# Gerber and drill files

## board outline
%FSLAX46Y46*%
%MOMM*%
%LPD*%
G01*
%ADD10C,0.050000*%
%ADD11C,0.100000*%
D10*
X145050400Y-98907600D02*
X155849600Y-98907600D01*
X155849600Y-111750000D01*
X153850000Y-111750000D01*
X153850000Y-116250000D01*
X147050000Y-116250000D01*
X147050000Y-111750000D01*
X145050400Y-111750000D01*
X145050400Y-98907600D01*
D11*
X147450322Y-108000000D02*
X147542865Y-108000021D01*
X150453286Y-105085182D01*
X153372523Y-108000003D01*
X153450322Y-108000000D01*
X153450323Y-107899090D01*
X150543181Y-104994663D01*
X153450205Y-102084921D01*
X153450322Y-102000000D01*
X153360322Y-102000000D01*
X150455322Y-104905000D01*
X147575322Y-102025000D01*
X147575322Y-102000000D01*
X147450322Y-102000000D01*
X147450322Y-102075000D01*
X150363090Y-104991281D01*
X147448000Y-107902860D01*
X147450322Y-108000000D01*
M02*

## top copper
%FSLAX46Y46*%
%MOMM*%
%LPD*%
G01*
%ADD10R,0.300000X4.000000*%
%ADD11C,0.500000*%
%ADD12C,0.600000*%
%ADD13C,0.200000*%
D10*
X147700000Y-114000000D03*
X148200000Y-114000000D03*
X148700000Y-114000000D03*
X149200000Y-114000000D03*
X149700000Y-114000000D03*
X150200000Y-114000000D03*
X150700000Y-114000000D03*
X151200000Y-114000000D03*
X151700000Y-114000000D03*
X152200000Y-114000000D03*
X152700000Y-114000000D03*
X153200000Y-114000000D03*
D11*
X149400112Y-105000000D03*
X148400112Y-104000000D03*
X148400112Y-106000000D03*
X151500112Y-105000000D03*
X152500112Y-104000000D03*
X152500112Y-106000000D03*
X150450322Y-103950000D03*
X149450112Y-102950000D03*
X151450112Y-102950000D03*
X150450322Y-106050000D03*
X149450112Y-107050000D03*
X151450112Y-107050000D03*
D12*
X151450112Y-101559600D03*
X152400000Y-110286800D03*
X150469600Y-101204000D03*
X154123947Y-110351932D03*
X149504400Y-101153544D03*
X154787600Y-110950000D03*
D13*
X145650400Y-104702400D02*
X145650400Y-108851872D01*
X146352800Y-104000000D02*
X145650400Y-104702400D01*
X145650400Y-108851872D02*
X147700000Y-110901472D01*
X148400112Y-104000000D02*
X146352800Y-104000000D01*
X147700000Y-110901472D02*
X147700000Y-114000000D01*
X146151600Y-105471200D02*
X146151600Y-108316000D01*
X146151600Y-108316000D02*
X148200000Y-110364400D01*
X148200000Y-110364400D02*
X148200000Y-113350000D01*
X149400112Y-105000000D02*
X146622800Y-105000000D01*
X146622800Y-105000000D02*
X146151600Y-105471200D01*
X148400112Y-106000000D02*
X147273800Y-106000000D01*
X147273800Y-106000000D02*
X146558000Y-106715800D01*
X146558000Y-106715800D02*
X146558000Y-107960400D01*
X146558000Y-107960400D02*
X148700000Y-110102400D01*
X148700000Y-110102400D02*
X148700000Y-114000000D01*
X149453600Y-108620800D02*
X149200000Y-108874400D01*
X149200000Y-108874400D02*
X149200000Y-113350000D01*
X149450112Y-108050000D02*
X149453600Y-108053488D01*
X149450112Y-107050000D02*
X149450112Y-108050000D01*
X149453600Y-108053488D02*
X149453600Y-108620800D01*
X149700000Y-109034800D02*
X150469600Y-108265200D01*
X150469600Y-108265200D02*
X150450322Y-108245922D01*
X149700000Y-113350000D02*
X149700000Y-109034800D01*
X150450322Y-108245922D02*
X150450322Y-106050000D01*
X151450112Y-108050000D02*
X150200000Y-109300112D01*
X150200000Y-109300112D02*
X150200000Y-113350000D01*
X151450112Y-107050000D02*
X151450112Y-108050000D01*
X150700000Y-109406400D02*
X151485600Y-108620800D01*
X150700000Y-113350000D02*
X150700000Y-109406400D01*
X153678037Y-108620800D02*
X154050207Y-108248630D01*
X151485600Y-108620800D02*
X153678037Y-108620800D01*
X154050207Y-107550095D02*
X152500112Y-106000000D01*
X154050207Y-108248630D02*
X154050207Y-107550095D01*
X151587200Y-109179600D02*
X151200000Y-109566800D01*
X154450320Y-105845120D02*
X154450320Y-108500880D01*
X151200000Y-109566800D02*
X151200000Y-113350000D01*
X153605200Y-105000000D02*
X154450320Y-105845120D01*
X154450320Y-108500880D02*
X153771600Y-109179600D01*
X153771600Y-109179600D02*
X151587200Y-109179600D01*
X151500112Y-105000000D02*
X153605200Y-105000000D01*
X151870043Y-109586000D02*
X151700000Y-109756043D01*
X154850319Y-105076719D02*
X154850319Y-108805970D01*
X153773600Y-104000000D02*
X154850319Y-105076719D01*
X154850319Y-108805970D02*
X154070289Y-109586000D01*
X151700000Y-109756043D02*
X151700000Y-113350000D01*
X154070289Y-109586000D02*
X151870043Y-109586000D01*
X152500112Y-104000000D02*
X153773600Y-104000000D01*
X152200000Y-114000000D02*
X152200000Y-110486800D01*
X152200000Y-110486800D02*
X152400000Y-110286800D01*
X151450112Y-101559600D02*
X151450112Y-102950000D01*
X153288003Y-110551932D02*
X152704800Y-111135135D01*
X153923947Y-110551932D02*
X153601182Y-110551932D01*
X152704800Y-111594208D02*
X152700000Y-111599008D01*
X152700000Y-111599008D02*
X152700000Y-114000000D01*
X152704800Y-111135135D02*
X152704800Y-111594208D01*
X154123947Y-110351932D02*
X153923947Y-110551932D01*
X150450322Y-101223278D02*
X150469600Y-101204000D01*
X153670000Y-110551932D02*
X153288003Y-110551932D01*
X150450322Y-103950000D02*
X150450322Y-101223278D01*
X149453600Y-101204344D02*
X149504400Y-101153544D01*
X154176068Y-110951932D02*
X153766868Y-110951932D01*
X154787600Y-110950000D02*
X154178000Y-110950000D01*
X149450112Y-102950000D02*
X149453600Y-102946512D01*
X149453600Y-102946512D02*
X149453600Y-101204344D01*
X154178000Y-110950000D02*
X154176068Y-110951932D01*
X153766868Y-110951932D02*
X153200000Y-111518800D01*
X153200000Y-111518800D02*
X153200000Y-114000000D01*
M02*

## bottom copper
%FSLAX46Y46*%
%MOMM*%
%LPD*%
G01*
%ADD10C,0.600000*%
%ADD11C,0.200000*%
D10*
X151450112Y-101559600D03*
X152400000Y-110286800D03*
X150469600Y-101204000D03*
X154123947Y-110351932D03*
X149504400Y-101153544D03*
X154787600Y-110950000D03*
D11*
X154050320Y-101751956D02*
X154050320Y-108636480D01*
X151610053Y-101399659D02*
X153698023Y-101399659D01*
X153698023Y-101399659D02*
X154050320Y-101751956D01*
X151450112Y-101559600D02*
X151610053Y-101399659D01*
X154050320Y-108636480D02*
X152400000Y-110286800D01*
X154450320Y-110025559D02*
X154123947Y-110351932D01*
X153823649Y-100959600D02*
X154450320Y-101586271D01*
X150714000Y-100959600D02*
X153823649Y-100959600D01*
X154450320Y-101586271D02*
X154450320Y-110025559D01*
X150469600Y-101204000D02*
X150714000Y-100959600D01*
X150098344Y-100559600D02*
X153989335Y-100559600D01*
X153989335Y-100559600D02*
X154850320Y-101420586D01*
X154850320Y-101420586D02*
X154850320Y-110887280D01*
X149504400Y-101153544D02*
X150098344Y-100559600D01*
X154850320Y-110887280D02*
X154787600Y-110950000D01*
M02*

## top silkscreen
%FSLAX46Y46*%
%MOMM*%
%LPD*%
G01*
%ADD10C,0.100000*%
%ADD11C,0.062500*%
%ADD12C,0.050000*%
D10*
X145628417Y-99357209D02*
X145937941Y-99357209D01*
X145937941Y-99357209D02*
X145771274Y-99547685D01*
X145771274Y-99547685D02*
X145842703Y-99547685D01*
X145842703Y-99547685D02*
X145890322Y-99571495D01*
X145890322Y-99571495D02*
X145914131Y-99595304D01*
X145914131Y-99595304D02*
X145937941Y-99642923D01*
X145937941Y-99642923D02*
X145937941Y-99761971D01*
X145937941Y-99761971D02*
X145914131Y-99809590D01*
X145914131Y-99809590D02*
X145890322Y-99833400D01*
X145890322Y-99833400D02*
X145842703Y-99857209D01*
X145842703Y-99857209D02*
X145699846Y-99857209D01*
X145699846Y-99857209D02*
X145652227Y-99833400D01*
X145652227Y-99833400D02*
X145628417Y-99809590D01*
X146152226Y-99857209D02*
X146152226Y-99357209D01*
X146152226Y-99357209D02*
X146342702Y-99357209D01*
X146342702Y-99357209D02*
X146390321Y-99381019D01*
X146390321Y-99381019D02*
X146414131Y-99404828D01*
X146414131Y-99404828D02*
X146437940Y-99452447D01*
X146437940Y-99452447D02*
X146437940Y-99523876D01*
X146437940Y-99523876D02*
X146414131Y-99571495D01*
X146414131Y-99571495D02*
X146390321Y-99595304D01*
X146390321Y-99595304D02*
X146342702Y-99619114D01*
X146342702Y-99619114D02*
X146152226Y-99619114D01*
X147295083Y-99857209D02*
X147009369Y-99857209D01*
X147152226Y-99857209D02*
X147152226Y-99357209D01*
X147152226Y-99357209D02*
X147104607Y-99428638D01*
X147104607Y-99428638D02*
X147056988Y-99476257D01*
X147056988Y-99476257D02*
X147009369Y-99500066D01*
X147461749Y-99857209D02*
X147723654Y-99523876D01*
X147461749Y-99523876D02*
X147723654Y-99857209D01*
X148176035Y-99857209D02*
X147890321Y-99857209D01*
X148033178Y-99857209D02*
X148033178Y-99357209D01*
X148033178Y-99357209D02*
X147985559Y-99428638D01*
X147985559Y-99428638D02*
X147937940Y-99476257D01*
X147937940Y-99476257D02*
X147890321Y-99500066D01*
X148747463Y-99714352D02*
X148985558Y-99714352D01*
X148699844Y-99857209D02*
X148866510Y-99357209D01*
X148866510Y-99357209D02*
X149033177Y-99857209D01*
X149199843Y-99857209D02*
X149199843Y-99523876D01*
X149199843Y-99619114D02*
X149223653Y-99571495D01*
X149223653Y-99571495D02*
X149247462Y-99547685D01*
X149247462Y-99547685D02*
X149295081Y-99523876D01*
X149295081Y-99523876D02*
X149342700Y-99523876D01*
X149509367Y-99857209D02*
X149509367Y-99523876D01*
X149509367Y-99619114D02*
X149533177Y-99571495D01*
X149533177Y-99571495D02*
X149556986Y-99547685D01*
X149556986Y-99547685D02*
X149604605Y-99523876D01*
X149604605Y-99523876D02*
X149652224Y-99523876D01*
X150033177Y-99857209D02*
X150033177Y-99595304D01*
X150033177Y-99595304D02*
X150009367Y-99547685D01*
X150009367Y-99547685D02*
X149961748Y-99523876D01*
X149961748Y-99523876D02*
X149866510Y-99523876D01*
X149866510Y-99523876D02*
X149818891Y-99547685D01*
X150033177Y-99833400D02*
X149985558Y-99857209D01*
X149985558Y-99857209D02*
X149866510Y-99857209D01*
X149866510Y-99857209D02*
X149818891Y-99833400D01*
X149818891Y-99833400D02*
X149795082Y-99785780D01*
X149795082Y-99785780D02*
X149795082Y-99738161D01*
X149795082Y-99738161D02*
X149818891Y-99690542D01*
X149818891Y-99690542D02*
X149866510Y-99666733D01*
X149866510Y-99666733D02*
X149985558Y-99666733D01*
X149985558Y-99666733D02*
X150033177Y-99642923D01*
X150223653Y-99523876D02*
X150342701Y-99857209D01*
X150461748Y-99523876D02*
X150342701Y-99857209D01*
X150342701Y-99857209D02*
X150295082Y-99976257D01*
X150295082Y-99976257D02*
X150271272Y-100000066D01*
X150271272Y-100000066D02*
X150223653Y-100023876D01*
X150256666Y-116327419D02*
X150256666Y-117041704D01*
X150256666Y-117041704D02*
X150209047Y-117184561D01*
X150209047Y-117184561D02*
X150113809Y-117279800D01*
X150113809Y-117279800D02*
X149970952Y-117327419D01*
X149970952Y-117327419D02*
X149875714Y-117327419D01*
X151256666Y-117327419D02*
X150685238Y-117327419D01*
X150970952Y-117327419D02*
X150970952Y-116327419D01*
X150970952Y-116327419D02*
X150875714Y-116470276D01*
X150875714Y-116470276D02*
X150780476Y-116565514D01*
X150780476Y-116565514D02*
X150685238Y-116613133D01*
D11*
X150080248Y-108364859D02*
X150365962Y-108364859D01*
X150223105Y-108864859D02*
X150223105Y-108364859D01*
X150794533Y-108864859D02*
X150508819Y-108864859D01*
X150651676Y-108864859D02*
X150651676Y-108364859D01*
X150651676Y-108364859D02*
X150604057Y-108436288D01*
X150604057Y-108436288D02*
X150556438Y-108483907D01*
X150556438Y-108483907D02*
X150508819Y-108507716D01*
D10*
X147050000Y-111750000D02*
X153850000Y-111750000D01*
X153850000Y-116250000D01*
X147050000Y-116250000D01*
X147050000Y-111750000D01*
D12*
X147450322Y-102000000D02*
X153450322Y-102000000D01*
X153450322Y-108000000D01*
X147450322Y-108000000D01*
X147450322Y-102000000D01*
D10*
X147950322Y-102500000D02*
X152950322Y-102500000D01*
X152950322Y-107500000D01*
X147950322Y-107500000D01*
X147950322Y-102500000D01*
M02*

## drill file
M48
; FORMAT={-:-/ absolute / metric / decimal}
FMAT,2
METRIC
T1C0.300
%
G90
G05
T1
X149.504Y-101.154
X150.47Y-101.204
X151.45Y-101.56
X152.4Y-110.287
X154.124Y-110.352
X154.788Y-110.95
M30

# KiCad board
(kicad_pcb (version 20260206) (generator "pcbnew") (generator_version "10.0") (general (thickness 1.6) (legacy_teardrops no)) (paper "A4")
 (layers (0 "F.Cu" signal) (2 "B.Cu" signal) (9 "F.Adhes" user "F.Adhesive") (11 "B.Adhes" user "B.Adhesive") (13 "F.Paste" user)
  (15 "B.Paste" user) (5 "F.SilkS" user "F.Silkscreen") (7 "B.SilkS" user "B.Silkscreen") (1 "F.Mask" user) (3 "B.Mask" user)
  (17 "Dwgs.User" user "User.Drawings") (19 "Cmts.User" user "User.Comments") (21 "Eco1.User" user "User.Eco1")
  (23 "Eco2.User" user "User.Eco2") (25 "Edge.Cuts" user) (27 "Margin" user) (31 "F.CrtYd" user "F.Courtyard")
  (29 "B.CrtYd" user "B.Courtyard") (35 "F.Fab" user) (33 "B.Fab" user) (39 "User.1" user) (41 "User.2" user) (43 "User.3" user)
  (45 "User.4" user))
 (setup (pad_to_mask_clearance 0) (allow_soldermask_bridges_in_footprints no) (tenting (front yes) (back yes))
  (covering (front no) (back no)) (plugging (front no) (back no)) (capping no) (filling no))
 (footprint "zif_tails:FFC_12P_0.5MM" (layer "F.Cu") (at 150.59 112)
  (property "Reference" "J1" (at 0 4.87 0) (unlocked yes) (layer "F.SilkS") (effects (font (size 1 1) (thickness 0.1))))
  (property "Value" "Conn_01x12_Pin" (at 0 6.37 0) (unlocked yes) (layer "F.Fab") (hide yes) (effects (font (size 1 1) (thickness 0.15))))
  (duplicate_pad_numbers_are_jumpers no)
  (fp_rect (start -3.54 -0.25) (end 3.26 4.25) (stroke (width 0.1) (type default)) (fill no) (layer "F.SilkS"))
  (pad "1" smd rect (at -2.89 2) (size 0.3 4) (layers "F.Cu" "F.Mask") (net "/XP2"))
  (pad "2" smd rect (at -2.39 2) (size 0.3 4) (layers "F.Cu" "F.Mask") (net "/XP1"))
  (pad "3" smd rect (at -1.89 2) (size 0.3 4) (layers "F.Cu" "F.Mask") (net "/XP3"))
  (pad "4" smd rect (at -1.39 2) (size 0.3 4) (layers "F.Cu" "F.Mask") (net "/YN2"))
  (pad "5" smd rect (at -0.89 2) (size 0.3 4) (layers "F.Cu" "F.Mask") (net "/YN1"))
  (pad "6" smd rect (at -0.39 2) (size 0.3 4) (layers "F.Cu" "F.Mask") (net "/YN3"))
  (pad "7" smd rect (at 0.11 2) (size 0.3 4) (layers "F.Cu" "F.Mask") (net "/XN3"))
  (pad "8" smd rect (at 0.61 2) (size 0.3 4) (layers "F.Cu" "F.Mask") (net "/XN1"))
  (pad "9" smd rect (at 1.11 2) (size 0.3 4) (layers "F.Cu" "F.Mask") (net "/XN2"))
  (pad "10" smd rect (at 1.61 2) (size 0.3 4) (layers "F.Cu" "F.Mask") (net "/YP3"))
  (pad "11" smd rect (at 2.11 2) (size 0.3 4) (layers "F.Cu" "F.Mask") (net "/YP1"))
  (pad "12" smd rect (at 2.61 2) (size 0.3 4) (layers "F.Cu" "F.Mask") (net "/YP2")))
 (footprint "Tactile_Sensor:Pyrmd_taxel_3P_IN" (layer "F.Cu") (at 150.450112 105)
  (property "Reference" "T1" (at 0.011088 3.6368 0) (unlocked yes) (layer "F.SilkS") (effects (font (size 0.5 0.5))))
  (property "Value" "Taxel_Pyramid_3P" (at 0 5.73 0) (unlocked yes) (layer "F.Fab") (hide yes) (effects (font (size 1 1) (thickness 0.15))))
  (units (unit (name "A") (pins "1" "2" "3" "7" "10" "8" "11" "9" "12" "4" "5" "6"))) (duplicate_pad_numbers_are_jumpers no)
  (fp_rect (start -2.99979 -3) (end 3.00021 3) (stroke (width 0.05) (type solid)) (fill no) (layer "F.SilkS"))
  (fp_rect (start -2.49979 -2.5) (end 2.50021 2.5) (stroke (width 0.1) (type solid)) (fill no) (layer "F.SilkS"))
  (fp_poly
   (pts (xy -2.99979 3) (xy -2.907247 3.000021) (xy 0.003174 0.085182) (xy 2.922411 3.000003) (xy 3.00021 3) (xy 3.000211 2.89909)
    (xy 0.093069 -0.005337) (xy 3.000093 -2.915079) (xy 3.00021 -3) (xy 2.91021 -3) (xy 0.00521 -0.095) (xy -2.87479 -2.975)
    (xy -2.87479 -3) (xy -2.99979 -3) (xy -2.99979 -2.925) (xy -0.087022 -0.008719) (xy -3.002112 2.90286))
   (stroke (width 0.1) (type solid)) (fill no) (layer "Edge.Cuts"))
  (pad "1" smd circle (at -1.05 0 270) (size 0.5 0.5) (layers "F.Cu" "F.Mask") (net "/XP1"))
  (pad "2" smd circle (at -2.05 -1 270) (size 0.5 0.5) (layers "F.Cu" "F.Mask") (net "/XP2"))
  (pad "3" smd circle (at -2.05 1 270) (size 0.5 0.5) (layers "F.Cu" "F.Mask") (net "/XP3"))
  (pad "4" smd circle (at 1.05 0 90) (size 0.5 0.5) (layers "F.Cu" "F.Mask" "F.Paste") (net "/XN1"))
  (pad "5" smd circle (at 2.05 -1 90) (size 0.5 0.5) (layers "F.Cu" "F.Mask" "F.Paste") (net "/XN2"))
  (pad "6" smd circle (at 2.05 1 90) (size 0.5 0.5) (layers "F.Cu" "F.Mask" "F.Paste") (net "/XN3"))
  (pad "7" smd circle (at 0.00021 -1.05) (size 0.5 0.5) (layers "F.Cu" "F.Mask") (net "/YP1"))
  (pad "8" smd circle (at -1 -2.05) (size 0.5 0.5) (layers "F.Cu" "F.Mask") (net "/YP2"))
  (pad "9" smd circle (at 1 -2.05) (size 0.5 0.5) (layers "F.Cu" "F.Mask") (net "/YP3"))
  (pad "10" smd circle (at 0.00021 1.05) (size 0.5 0.5) (layers "F.Cu" "F.Mask") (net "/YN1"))
  (pad "11" smd circle (at -1 2.05) (size 0.5 0.5) (layers "F.Cu" "F.Mask") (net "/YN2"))
  (pad "12" smd circle (at 1 2.05) (size 0.5 0.5) (layers "F.Cu" "F.Mask") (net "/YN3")))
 (gr_poly
  (pts (xy 145.0504 98.9076) (xy 155.8496 98.9076) (xy 155.8496 111.75) (xy 153.85 111.75) (xy 153.85 116.25) (xy 147.05 116.25)
   (xy 147.05 111.75) (xy 145.0504 111.75))
  (stroke (width 0.05) (type solid)) (fill no) (layer "Edge.Cuts"))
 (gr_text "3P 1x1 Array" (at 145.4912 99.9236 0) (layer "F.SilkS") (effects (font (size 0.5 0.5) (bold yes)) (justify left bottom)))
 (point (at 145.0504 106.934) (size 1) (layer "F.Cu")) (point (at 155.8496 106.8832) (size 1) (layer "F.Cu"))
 (segment (start 145.6504 104.7024) (end 145.6504 108.851872) (width 0.2) (layer "F.Cu") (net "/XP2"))
 (segment (start 146.3528 104) (end 145.6504 104.7024) (width 0.2) (layer "F.Cu") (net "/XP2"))
 (segment (start 145.6504 108.851872) (end 147.7 110.901472) (width 0.2) (layer "F.Cu") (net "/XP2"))
 (segment (start 148.400112 104) (end 146.3528 104) (width 0.2) (layer "F.Cu") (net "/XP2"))
 (segment (start 147.7 110.901472) (end 147.7 114) (width 0.2) (layer "F.Cu") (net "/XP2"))
 (segment (start 146.1516 105.4712) (end 146.1516 108.316) (width 0.2) (layer "F.Cu") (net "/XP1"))
 (segment (start 146.1516 108.316) (end 148.2 110.3644) (width 0.2) (layer "F.Cu") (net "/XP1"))
 (segment (start 148.2 110.3644) (end 148.2 113.35) (width 0.2) (layer "F.Cu") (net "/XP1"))
 (segment (start 149.400112 105) (end 146.6228 105) (width 0.2) (layer "F.Cu") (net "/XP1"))
 (segment (start 146.6228 105) (end 146.1516 105.4712) (width 0.2) (layer "F.Cu") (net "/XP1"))
 (segment (start 148.400112 106) (end 147.2738 106) (width 0.2) (layer "F.Cu") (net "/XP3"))
 (segment (start 147.2738 106) (end 146.558 106.7158) (width 0.2) (layer "F.Cu") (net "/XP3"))
 (segment (start 146.558 106.7158) (end 146.558 107.9604) (width 0.2) (layer "F.Cu") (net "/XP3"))
 (segment (start 146.558 107.9604) (end 148.7 110.1024) (width 0.2) (layer "F.Cu") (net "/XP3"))
 (segment (start 148.7 110.1024) (end 148.7 114) (width 0.2) (layer "F.Cu") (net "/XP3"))
 (segment (start 149.4536 108.6208) (end 149.2 108.8744) (width 0.2) (layer "F.Cu") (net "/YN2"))
 (segment (start 149.2 108.8744) (end 149.2 113.35) (width 0.2) (layer "F.Cu") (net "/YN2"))
 (segment (start 149.450112 108.05) (end 149.4536 108.053488) (width 0.2) (layer "F.Cu") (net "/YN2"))
 (segment (start 149.450112 107.05) (end 149.450112 108.05) (width 0.2) (layer "F.Cu") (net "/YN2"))
 (segment (start 149.4536 108.053488) (end 149.4536 108.6208) (width 0.2) (layer "F.Cu") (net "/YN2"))
 (segment (start 149.7 109.0348) (end 150.4696 108.2652) (width 0.2) (layer "F.Cu") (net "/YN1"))
 (segment (start 150.4696 108.2652) (end 150.450322 108.245922) (width 0.2) (layer "F.Cu") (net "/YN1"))
 (segment (start 149.7 113.35) (end 149.7 109.0348) (width 0.2) (layer "F.Cu") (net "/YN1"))
 (segment (start 150.450322 108.245922) (end 150.450322 106.05) (width 0.2) (layer "F.Cu") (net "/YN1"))
 (segment (start 151.450112 108.05) (end 150.2 109.300112) (width 0.2) (layer "F.Cu") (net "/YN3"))
 (segment (start 150.2 109.300112) (end 150.2 113.35) (width 0.2) (layer "F.Cu") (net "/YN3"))
 (segment (start 151.450112 107.05) (end 151.450112 108.05) (width 0.2) (layer "F.Cu") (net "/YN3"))
 (segment (start 150.7 109.4064) (end 151.4856 108.6208) (width 0.2) (layer "F.Cu") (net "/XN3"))
 (segment (start 150.7 113.35) (end 150.7 109.4064) (width 0.2) (layer "F.Cu") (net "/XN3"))
 (segment (start 153.678037 108.6208) (end 154.050207 108.24863) (width 0.2) (layer "F.Cu") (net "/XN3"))
 (segment (start 151.4856 108.6208) (end 153.678037 108.6208) (width 0.2) (layer "F.Cu") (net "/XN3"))
 (segment (start 154.050207 107.550095) (end 152.500112 106) (width 0.2) (layer "F.Cu") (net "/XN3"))
 (segment (start 154.050207 108.24863) (end 154.050207 107.550095) (width 0.2) (layer "F.Cu") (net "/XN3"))
 (segment (start 151.5872 109.1796) (end 151.2 109.5668) (width 0.2) (layer "F.Cu") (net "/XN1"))
 (segment (start 154.45032 105.84512) (end 154.45032 108.50088) (width 0.2) (layer "F.Cu") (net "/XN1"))
 (segment (start 151.2 109.5668) (end 151.2 113.35) (width 0.2) (layer "F.Cu") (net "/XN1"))
 (segment (start 153.6052 105) (end 154.45032 105.84512) (width 0.2) (layer "F.Cu") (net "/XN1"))
 (segment (start 154.45032 108.50088) (end 153.7716 109.1796) (width 0.2) (layer "F.Cu") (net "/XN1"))
 (segment (start 153.7716 109.1796) (end 151.5872 109.1796) (width 0.2) (layer "F.Cu") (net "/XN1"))
 (segment (start 151.500112 105) (end 153.6052 105) (width 0.2) (layer "F.Cu") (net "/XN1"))
 (segment (start 151.870043 109.586) (end 151.7 109.756043) (width 0.2) (layer "F.Cu") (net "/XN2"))
 (segment (start 154.850319 105.076719) (end 154.850319 108.80597) (width 0.2) (layer "F.Cu") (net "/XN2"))
 (segment (start 153.7736 104) (end 154.850319 105.076719) (width 0.2) (layer "F.Cu") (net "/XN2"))
 (segment (start 154.850319 108.80597) (end 154.070289 109.586) (width 0.2) (layer "F.Cu") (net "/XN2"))
 (segment (start 151.7 109.756043) (end 151.7 113.35) (width 0.2) (layer "F.Cu") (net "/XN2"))
 (segment (start 154.070289 109.586) (end 151.870043 109.586) (width 0.2) (layer "F.Cu") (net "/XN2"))
 (segment (start 152.500112 104) (end 153.7736 104) (width 0.2) (layer "F.Cu") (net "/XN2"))
 (segment (start 152.2 114) (end 152.2 110.4868) (width 0.2) (layer "F.Cu") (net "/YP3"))
 (segment (start 152.2 110.4868) (end 152.4 110.2868) (width 0.2) (layer "F.Cu") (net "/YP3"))
 (segment (start 151.450112 101.5596) (end 151.450112 102.95) (width 0.2) (layer "F.Cu") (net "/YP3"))
 (via (at 151.450112 101.5596) (size 0.6) (drill 0.3) (layers "F.Cu" "B.Cu") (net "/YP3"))
 (via (at 152.4 110.2868) (size 0.6) (drill 0.3) (layers "F.Cu" "B.Cu") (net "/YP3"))
 (segment (start 154.05032 101.751956) (end 154.05032 108.63648) (width 0.2) (layer "B.Cu") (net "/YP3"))
 (segment (start 151.610053 101.399659) (end 153.698023 101.399659) (width 0.2) (layer "B.Cu") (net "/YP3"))
 (segment (start 153.698023 101.399659) (end 154.05032 101.751956) (width 0.2) (layer "B.Cu") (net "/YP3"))
 (segment (start 151.450112 101.5596) (end 151.610053 101.399659) (width 0.2) (layer "B.Cu") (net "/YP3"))
 (segment (start 154.05032 108.63648) (end 152.4 110.2868) (width 0.2) (layer "B.Cu") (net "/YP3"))
 (segment (start 153.288003 110.551932) (end 152.7048 111.135135) (width 0.2) (layer "F.Cu") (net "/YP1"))
 (segment (start 153.923947 110.551932) (end 153.601182 110.551932) (width 0.2) (layer "F.Cu") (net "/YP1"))
 (segment (start 152.7048 111.594208) (end 152.7 111.599008) (width 0.2) (layer "F.Cu") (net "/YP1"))
 (segment (start 152.7 111.599008) (end 152.7 114) (width 0.2) (layer "F.Cu") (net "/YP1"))
 (segment (start 152.7048 111.135135) (end 152.7048 111.594208) (width 0.2) (layer "F.Cu") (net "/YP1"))
 (segment (start 154.123947 110.351932) (end 153.923947 110.551932) (width 0.2) (layer "F.Cu") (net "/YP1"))
 (segment (start 150.450322 101.223278) (end 150.4696 101.204) (width 0.2) (layer "F.Cu") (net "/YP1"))
 (segment (start 153.67 110.551932) (end 153.288003 110.551932) (width 0.2) (layer "F.Cu") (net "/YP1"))
 (segment (start 150.450322 103.95) (end 150.450322 101.223278) (width 0.2) (layer "F.Cu") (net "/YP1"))
 (via (at 150.4696 101.204) (size 0.6) (drill 0.3) (layers "F.Cu" "B.Cu") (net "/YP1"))
 (via (at 154.123947 110.351932) (size 0.6) (drill 0.3) (layers "F.Cu" "B.Cu") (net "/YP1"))
 (segment (start 154.45032 110.025559) (end 154.123947 110.351932) (width 0.2) (layer "B.Cu") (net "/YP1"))
 (segment (start 153.823649 100.9596) (end 154.45032 101.586271) (width 0.2) (layer "B.Cu") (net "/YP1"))
 (segment (start 150.714 100.9596) (end 153.823649 100.9596) (width 0.2) (layer "B.Cu") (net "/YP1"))
 (segment (start 154.45032 101.586271) (end 154.45032 110.025559) (width 0.2) (layer "B.Cu") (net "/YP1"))
 (segment (start 150.4696 101.204) (end 150.714 100.9596) (width 0.2) (layer "B.Cu") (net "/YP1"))
 (segment (start 149.4536 101.204344) (end 149.5044 101.153544) (width 0.2) (layer "F.Cu") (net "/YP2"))
 (segment (start 154.176068 110.951932) (end 153.766868 110.951932) (width 0.2) (layer "F.Cu") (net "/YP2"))
 (segment (start 154.7876 110.95) (end 154.178 110.95) (width 0.2) (layer "F.Cu") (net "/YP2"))
 (segment (start 149.450112 102.95) (end 149.4536 102.946512) (width 0.2) (layer "F.Cu") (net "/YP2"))
 (segment (start 149.4536 102.946512) (end 149.4536 101.204344) (width 0.2) (layer "F.Cu") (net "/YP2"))
 (segment (start 154.178 110.95) (end 154.176068 110.951932) (width 0.2) (layer "F.Cu") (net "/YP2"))
 (segment (start 153.766868 110.951932) (end 153.2 111.5188) (width 0.2) (layer "F.Cu") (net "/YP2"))
 (segment (start 153.2 111.5188) (end 153.2 114) (width 0.2) (layer "F.Cu") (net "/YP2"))
 (via (at 149.5044 101.153544) (size 0.6) (drill 0.3) (layers "F.Cu" "B.Cu") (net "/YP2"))
 (via (at 154.7876 110.95) (size 0.6) (drill 0.3) (layers "F.Cu" "B.Cu") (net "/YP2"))
 (segment (start 150.098344 100.5596) (end 153.989335 100.5596) (width 0.2) (layer "B.Cu") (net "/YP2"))
 (segment (start 153.989335 100.5596) (end 154.85032 101.420586) (width 0.2) (layer "B.Cu") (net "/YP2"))
 (segment (start 154.85032 101.420586) (end 154.85032 110.88728) (width 0.2) (layer "B.Cu") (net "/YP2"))
 (segment (start 149.5044 101.153544) (end 150.098344 100.5596) (width 0.2) (layer "B.Cu") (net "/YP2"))
 (segment (start 154.85032 110.88728) (end 154.7876 110.95) (width 0.2) (layer "B.Cu") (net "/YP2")))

